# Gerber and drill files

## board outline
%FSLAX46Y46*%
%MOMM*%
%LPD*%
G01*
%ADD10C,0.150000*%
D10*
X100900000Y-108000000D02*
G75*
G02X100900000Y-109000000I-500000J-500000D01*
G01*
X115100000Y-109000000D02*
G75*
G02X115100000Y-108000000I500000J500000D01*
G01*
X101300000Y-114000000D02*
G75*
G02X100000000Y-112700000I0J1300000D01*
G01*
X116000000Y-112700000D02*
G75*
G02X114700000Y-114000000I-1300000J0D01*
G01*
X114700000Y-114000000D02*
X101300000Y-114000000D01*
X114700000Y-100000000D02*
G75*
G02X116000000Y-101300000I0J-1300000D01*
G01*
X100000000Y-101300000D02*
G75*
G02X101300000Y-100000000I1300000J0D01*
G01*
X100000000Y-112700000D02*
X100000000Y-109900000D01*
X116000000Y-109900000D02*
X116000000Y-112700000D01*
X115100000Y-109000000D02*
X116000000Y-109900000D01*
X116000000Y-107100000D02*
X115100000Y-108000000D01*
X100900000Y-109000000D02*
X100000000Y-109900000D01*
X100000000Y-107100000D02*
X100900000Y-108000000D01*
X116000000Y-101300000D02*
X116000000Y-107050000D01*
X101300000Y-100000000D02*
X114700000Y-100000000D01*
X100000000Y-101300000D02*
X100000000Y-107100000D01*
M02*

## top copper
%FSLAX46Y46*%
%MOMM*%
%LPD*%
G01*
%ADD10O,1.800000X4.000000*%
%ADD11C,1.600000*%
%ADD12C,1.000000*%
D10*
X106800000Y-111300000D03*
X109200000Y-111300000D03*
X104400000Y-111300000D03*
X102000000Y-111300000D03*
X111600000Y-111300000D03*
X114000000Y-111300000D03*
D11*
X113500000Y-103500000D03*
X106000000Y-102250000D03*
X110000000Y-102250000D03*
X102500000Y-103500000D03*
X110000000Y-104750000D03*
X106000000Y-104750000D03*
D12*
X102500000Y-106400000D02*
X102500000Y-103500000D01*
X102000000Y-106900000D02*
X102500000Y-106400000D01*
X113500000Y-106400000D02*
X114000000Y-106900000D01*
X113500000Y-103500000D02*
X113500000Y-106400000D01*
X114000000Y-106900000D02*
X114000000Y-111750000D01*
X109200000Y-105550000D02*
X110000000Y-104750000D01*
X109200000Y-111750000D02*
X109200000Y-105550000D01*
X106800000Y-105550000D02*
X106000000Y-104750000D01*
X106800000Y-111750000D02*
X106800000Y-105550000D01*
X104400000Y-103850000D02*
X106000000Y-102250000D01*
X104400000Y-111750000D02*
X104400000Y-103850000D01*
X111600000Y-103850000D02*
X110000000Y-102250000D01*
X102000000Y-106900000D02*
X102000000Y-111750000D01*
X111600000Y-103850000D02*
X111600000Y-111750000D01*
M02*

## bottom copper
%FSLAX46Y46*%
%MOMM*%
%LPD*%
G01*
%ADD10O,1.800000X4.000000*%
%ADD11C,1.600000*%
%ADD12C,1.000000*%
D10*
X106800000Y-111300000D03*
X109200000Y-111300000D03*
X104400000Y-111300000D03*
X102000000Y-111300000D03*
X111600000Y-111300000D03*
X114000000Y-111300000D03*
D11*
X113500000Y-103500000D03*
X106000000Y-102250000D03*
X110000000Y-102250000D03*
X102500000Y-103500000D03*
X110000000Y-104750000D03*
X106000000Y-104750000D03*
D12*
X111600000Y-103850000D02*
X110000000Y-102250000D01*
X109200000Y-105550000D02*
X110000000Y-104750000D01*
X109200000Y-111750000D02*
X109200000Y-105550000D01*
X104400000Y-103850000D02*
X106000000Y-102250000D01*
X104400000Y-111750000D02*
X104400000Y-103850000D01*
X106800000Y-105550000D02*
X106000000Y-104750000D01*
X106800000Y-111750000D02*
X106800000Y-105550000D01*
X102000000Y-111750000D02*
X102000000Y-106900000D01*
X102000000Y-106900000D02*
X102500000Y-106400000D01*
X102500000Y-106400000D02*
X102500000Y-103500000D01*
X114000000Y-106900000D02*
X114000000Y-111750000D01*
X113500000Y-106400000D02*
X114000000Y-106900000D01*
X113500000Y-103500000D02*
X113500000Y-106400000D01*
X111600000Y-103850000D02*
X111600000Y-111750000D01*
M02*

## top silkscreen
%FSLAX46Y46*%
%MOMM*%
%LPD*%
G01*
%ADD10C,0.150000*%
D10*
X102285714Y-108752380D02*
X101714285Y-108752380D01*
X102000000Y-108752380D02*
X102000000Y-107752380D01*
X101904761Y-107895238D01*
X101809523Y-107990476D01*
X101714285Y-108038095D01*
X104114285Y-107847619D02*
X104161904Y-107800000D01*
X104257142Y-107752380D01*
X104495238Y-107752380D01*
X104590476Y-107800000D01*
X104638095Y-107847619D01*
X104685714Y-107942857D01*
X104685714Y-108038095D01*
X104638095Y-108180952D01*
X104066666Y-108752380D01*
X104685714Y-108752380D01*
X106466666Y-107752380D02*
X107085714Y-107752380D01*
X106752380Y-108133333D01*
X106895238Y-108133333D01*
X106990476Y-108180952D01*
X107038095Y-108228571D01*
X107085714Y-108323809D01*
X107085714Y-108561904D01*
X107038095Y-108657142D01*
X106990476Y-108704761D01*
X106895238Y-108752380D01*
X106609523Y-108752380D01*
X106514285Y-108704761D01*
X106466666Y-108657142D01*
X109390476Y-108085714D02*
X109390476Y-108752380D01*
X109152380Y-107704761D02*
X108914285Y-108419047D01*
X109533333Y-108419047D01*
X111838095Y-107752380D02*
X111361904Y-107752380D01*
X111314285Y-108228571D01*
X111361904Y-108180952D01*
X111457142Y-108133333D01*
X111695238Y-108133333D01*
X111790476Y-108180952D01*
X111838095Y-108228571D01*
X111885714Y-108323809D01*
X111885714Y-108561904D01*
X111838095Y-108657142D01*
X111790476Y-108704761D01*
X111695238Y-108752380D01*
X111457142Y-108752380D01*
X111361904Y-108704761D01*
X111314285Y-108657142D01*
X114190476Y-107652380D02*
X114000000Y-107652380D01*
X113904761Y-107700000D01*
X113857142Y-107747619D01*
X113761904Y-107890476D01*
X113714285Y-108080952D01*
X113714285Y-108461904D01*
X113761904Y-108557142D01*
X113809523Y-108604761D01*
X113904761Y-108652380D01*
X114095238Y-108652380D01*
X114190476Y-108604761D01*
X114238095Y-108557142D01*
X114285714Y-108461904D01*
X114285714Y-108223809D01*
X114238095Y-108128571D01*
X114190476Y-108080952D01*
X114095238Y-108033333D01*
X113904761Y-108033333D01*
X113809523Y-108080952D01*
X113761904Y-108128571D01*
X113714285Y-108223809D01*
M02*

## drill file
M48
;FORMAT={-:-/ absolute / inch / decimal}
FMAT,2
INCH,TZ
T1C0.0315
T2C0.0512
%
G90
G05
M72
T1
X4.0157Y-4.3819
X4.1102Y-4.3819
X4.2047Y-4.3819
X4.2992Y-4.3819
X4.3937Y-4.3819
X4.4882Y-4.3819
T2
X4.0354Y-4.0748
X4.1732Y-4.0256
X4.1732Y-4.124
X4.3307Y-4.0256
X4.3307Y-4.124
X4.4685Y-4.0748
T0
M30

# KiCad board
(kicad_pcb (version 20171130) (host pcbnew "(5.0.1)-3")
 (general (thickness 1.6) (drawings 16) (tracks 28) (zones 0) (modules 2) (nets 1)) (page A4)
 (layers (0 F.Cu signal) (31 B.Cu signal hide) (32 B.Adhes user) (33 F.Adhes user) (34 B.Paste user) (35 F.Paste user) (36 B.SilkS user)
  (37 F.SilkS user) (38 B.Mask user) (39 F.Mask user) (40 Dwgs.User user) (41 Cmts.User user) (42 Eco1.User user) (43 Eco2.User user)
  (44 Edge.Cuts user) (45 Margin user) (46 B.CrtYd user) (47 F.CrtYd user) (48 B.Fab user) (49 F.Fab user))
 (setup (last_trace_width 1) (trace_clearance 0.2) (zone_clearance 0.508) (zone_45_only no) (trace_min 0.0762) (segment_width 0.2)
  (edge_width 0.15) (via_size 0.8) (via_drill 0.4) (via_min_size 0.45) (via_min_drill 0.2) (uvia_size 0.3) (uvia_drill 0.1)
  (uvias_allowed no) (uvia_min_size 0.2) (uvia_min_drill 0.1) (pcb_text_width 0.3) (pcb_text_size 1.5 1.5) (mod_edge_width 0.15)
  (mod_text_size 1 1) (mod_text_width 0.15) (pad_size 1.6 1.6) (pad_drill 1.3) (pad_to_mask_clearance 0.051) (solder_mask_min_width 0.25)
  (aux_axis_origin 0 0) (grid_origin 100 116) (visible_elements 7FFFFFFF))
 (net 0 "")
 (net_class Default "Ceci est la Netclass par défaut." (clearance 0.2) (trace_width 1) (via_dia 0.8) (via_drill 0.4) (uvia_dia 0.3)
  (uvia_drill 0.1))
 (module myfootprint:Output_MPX (layer F.Cu) (at 108 111.3)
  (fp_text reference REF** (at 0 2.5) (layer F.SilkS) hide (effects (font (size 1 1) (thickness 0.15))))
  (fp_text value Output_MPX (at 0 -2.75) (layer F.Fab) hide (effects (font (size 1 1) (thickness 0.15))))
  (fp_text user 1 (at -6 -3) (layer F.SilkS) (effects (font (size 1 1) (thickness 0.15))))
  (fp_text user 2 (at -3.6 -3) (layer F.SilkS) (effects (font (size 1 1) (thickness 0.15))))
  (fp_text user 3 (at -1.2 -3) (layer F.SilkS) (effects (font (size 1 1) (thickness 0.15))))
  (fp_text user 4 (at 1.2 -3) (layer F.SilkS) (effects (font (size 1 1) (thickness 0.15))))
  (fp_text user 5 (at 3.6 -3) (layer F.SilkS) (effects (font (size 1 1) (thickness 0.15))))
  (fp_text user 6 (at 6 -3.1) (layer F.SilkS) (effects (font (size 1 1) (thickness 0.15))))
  (pad 3 thru_hole oval (at -1.2 0) (size 1.8 4) (drill 0.8) (layers *.Cu *.Mask))
  (pad 4 thru_hole oval (at 1.2 0) (size 1.8 4) (drill 0.8) (layers *.Cu *.Mask))
  (pad 2 thru_hole oval (at -3.6 0) (size 1.8 4) (drill 0.8) (layers *.Cu *.Mask))
  (pad 1 thru_hole oval (at -6 0) (size 1.8 4) (drill 0.8) (layers *.Cu *.Mask))
  (pad 5 thru_hole oval (at 3.6 0) (size 1.8 4) (drill 0.8) (layers *.Cu *.Mask))
  (pad 6 thru_hole oval (at 6 0) (size 1.8 4) (drill 0.8) (layers *.Cu *.Mask)))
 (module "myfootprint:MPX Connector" (layer F.Cu) (at 108 103.5)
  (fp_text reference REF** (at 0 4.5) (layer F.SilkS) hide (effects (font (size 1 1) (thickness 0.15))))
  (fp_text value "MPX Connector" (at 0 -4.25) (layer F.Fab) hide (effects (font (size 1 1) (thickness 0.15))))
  (pad 6 thru_hole circle (at 5.5 0) (size 1.6 1.6) (drill 1.3) (layers *.Cu *.Mask))
  (pad 2 thru_hole circle (at -2 -1.25) (size 1.6 1.6) (drill 1.3) (layers *.Cu *.Mask))
  (pad 4 thru_hole circle (at 2 -1.25) (size 1.6 1.6) (drill 1.3) (layers *.Cu *.Mask))
  (pad 1 thru_hole circle (at -5.5 0) (size 1.6 1.6) (drill 1.3) (layers *.Cu *.Mask))
  (pad 5 thru_hole circle (at 2 1.25) (size 1.6 1.6) (drill 1.3) (layers *.Cu *.Mask))
  (pad 3 thru_hole circle (at -2 1.25) (size 1.6 1.6) (drill 1.3) (layers *.Cu *.Mask)))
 (gr_arc (start 100.4 108.5) (end 100.9 109) (angle -90) (layer Edge.Cuts) (width 0.15))
 (gr_arc (start 115.6 108.5) (end 115.1 108) (angle -90) (layer Edge.Cuts) (width 0.15))
 (gr_arc (start 101.3 112.7) (end 100 112.7) (angle -90) (layer Edge.Cuts) (width 0.15))
 (gr_arc (start 114.7 112.7) (end 114.7 114) (angle -90) (layer Edge.Cuts) (width 0.15))
 (gr_line (start 114.7 114) (end 101.3 114) (layer Edge.Cuts) (width 0.15))
 (gr_arc (start 114.7 101.3) (end 116 101.3) (angle -90) (layer Edge.Cuts) (width 0.15))
 (gr_arc (start 101.3 101.3) (end 101.3 100) (angle -90) (layer Edge.Cuts) (width 0.15))
 (gr_line (start 100 112.7) (end 100 109.9) (layer Edge.Cuts) (width 0.15))
 (gr_line (start 116 109.9) (end 116 112.7) (layer Edge.Cuts) (width 0.15))
 (gr_line (start 115.1 109) (end 116 109.9) (layer Edge.Cuts) (width 0.15))
 (gr_line (start 116 107.1) (end 115.1 108) (layer Edge.Cuts) (width 0.15))
 (gr_line (start 100.9 109) (end 100 109.9) (layer Edge.Cuts) (width 0.15))
 (gr_line (start 100 107.1) (end 100.9 108) (layer Edge.Cuts) (width 0.15))
 (gr_line (start 116 101.3) (end 116 107.05) (layer Edge.Cuts) (width 0.15))
 (gr_line (start 101.3 100) (end 114.7 100) (layer Edge.Cuts) (width 0.15))
 (gr_line (start 100 101.3) (end 100 107.1) (layer Edge.Cuts) (width 0.15))
 (segment (start 109.2 105.55) (end 110 104.75) (width 1) (layer F.Cu) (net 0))
 (segment (start 109.2 111.75) (end 109.2 105.55) (width 1) (layer F.Cu) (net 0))
 (segment (start 106.8 105.55) (end 106 104.75) (width 1) (layer F.Cu) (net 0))
 (segment (start 106.8 111.75) (end 106.8 105.55) (width 1) (layer F.Cu) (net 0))
 (segment (start 104.4 103.85) (end 106 102.25) (width 1) (layer F.Cu) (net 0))
 (segment (start 104.4 111.75) (end 104.4 103.85) (width 1) (layer F.Cu) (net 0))
 (segment (start 111.6 103.85) (end 110 102.25) (width 1) (layer F.Cu) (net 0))
 (segment (start 111.6 103.85) (end 110 102.25) (width 1) (layer B.Cu) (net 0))
 (segment (start 109.2 105.55) (end 110 104.75) (width 1) (layer B.Cu) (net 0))
 (segment (start 109.2 111.75) (end 109.2 105.55) (width 1) (layer B.Cu) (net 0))
 (segment (start 104.4 103.85) (end 106 102.25) (width 1) (layer B.Cu) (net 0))
 (segment (start 104.4 111.75) (end 104.4 103.85) (width 1) (layer B.Cu) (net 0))
 (segment (start 106.8 105.55) (end 106 104.75) (width 1) (layer B.Cu) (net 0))
 (segment (start 106.8 111.75) (end 106.8 105.55) (width 1) (layer B.Cu) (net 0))
 (segment (start 102 111.75) (end 102 106.9) (width 1) (layer B.Cu) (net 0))
 (segment (start 102 106.9) (end 102.5 106.4) (width 1) (layer B.Cu) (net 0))
 (segment (start 102.5 106.4) (end 102.5 103.5) (width 1) (layer B.Cu) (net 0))
 (segment (start 114 106.9) (end 114 111.75) (width 1) (layer B.Cu) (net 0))
 (segment (start 113.5 106.4) (end 114 106.9) (width 1) (layer B.Cu) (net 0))
 (segment (start 113.5 103.5) (end 113.5 106.4) (width 1) (layer B.Cu) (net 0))
 (segment (start 111.6 103.85) (end 111.6 111.75) (width 1) (layer F.Cu) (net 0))
 (segment (start 111.6 103.85) (end 111.6 111.75) (width 1) (layer B.Cu) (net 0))
 (segment (start 102 106.9) (end 102 111.75) (width 1) (layer F.Cu) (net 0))
 (segment (start 102 106.9) (end 102.5 106.4) (width 1) (layer F.Cu) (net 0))
 (segment (start 102.5 106.4) (end 102.5 103.5) (width 1) (layer F.Cu) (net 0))
 (segment (start 113.5 106.4) (end 114 106.9) (width 1) (layer F.Cu) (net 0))
 (segment (start 114 106.9) (end 114 111.75) (width 1) (layer F.Cu) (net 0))
 (segment (start 113.5 103.5) (end 113.5 106.4) (width 1) (layer F.Cu) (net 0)))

